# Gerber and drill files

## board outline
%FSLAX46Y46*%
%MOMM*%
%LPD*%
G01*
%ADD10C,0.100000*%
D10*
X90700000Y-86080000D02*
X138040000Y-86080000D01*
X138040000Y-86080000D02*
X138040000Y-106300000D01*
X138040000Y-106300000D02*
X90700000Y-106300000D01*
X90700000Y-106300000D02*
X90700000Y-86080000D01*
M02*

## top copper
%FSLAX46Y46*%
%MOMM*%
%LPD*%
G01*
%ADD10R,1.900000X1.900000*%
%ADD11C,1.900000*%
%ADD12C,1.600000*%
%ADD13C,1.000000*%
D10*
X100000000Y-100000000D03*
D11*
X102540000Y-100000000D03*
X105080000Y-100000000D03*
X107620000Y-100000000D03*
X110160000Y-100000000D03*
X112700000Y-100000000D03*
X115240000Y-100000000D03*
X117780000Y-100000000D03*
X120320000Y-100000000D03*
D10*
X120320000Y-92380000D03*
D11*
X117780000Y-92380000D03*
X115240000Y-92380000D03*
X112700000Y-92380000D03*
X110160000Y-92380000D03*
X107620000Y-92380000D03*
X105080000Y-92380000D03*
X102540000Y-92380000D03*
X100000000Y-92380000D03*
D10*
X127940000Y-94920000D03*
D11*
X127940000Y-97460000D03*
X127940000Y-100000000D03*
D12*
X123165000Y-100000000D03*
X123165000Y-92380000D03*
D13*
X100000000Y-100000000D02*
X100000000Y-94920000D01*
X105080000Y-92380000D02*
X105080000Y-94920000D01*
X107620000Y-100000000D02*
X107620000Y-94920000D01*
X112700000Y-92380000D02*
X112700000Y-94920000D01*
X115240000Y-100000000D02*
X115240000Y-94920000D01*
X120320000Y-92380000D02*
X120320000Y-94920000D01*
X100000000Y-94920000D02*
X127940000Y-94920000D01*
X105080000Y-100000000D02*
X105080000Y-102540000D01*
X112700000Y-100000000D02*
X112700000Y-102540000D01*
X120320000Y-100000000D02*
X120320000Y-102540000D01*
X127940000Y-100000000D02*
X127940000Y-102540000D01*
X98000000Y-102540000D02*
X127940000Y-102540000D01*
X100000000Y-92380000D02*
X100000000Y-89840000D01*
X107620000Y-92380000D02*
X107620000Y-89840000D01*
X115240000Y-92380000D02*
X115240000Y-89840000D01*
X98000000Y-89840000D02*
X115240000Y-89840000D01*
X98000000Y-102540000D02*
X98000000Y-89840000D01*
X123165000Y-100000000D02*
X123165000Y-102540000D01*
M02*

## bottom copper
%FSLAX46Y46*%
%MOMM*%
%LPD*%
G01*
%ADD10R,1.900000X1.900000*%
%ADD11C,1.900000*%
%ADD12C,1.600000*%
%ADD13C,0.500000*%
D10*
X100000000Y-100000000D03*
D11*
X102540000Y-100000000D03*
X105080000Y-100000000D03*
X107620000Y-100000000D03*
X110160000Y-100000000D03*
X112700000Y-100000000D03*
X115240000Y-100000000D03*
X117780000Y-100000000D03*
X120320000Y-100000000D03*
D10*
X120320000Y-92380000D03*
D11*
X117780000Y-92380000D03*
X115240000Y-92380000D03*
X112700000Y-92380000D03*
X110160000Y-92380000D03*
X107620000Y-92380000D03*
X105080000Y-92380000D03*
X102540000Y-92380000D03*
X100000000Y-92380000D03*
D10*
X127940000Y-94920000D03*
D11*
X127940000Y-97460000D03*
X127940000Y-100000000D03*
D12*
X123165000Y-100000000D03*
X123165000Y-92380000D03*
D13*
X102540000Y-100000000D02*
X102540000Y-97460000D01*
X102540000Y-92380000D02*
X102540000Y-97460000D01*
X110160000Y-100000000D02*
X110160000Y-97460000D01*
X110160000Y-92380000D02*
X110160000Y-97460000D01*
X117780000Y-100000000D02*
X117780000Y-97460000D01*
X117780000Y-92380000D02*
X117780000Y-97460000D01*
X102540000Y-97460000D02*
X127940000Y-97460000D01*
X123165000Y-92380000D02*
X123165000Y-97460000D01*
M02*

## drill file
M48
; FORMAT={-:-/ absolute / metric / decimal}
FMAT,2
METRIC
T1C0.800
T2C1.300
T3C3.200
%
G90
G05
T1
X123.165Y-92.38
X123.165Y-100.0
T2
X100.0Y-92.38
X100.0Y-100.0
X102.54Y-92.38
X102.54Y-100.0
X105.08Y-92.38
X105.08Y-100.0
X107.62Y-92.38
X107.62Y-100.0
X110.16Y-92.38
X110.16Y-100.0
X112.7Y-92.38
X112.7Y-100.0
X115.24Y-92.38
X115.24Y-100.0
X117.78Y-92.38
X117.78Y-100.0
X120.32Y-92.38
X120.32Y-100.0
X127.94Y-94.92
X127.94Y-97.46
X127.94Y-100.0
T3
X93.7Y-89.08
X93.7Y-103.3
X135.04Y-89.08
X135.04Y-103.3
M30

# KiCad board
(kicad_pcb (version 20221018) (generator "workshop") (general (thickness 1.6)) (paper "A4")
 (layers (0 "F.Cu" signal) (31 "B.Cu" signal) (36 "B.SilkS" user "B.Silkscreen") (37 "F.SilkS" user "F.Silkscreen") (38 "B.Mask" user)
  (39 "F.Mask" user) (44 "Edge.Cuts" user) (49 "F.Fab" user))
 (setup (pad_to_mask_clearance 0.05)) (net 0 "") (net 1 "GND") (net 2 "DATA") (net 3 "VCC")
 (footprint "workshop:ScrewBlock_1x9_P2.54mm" (layer "F.Cu") (at 100.000 100.000)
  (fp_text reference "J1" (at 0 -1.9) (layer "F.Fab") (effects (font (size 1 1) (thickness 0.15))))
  (pad "1" thru_hole rect (at 0.000 0) (size 1.9 1.9) (drill 1.3) (layers "*.Cu" "*.Mask") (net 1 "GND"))
  (pad "2" thru_hole circle (at 2.540 0) (size 1.9 1.9) (drill 1.3) (layers "*.Cu" "*.Mask") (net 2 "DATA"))
  (pad "3" thru_hole circle (at 5.080 0) (size 1.9 1.9) (drill 1.3) (layers "*.Cu" "*.Mask") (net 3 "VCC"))
  (pad "4" thru_hole circle (at 7.620 0) (size 1.9 1.9) (drill 1.3) (layers "*.Cu" "*.Mask") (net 1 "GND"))
  (pad "5" thru_hole circle (at 10.160 0) (size 1.9 1.9) (drill 1.3) (layers "*.Cu" "*.Mask") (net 2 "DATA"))
  (pad "6" thru_hole circle (at 12.700 0) (size 1.9 1.9) (drill 1.3) (layers "*.Cu" "*.Mask") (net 3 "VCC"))
  (pad "7" thru_hole circle (at 15.240 0) (size 1.9 1.9) (drill 1.3) (layers "*.Cu" "*.Mask") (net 1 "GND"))
  (pad "8" thru_hole circle (at 17.780 0) (size 1.9 1.9) (drill 1.3) (layers "*.Cu" "*.Mask") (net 2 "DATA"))
  (pad "9" thru_hole circle (at 20.320 0) (size 1.9 1.9) (drill 1.3) (layers "*.Cu" "*.Mask") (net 3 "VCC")))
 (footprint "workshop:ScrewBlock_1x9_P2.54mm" (layer "F.Cu") (at 120.320 92.380 180)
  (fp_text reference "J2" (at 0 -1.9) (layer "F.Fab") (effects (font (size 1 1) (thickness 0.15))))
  (pad "1" thru_hole rect (at 0.000 0) (size 1.9 1.9) (drill 1.3) (layers "*.Cu" "*.Mask") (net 1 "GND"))
  (pad "2" thru_hole circle (at 2.540 0) (size 1.9 1.9) (drill 1.3) (layers "*.Cu" "*.Mask") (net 2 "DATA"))
  (pad "3" thru_hole circle (at 5.080 0) (size 1.9 1.9) (drill 1.3) (layers "*.Cu" "*.Mask") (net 3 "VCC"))
  (pad "4" thru_hole circle (at 7.620 0) (size 1.9 1.9) (drill 1.3) (layers "*.Cu" "*.Mask") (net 1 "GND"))
  (pad "5" thru_hole circle (at 10.160 0) (size 1.9 1.9) (drill 1.3) (layers "*.Cu" "*.Mask") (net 2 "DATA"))
  (pad "6" thru_hole circle (at 12.700 0) (size 1.9 1.9) (drill 1.3) (layers "*.Cu" "*.Mask") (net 3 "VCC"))
  (pad "7" thru_hole circle (at 15.240 0) (size 1.9 1.9) (drill 1.3) (layers "*.Cu" "*.Mask") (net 1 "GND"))
  (pad "8" thru_hole circle (at 17.780 0) (size 1.9 1.9) (drill 1.3) (layers "*.Cu" "*.Mask") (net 2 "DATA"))
  (pad "9" thru_hole circle (at 20.320 0) (size 1.9 1.9) (drill 1.3) (layers "*.Cu" "*.Mask") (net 3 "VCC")))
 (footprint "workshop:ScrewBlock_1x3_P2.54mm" (layer "F.Cu") (at 127.940 94.920 270)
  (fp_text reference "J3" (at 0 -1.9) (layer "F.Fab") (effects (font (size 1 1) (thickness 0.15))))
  (pad "1" thru_hole rect (at 0.000 0) (size 1.9 1.9) (drill 1.3) (layers "*.Cu" "*.Mask") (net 1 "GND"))
  (pad "2" thru_hole circle (at 2.540 0) (size 1.9 1.9) (drill 1.3) (layers "*.Cu" "*.Mask") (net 2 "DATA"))
  (pad "3" thru_hole circle (at 5.080 0) (size 1.9 1.9) (drill 1.3) (layers "*.Cu" "*.Mask") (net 3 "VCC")))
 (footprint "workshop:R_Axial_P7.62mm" (layer "F.Cu") (at 123.165 100.000)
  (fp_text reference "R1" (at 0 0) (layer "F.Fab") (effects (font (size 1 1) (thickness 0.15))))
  (pad "1" thru_hole circle (at 0 0.000) (size 1.6 1.6) (drill 0.8) (layers "*.Cu" "*.Mask") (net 3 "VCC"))
  (pad "2" thru_hole circle (at 0 -7.620) (size 1.6 1.6) (drill 0.8) (layers "*.Cu" "*.Mask") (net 2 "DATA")))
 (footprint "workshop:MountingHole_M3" (layer "F.Cu") (at 93.700 89.080)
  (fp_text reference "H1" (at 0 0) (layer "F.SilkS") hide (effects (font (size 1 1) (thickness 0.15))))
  (pad "" np_thru_hole circle (at 0 0) (size 3.2 3.2) (drill 3.2) (layers "*.Cu" "*.Mask")))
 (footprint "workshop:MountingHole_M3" (layer "F.Cu") (at 93.700 103.300)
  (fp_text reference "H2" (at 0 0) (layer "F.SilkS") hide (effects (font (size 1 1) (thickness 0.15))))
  (pad "" np_thru_hole circle (at 0 0) (size 3.2 3.2) (drill 3.2) (layers "*.Cu" "*.Mask")))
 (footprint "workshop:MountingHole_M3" (layer "F.Cu") (at 135.040 89.080)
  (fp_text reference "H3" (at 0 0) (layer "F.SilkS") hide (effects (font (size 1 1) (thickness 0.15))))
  (pad "" np_thru_hole circle (at 0 0) (size 3.2 3.2) (drill 3.2) (layers "*.Cu" "*.Mask")))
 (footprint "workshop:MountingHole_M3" (layer "F.Cu") (at 135.040 103.300)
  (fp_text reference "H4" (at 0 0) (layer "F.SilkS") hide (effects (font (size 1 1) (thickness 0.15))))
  (pad "" np_thru_hole circle (at 0 0) (size 3.2 3.2) (drill 3.2) (layers "*.Cu" "*.Mask")))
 (segment (start 100.000 100.000) (end 100.000 94.920) (width 1.0) (layer "F.Cu") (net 1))
 (segment (start 105.080 92.380) (end 105.080 94.920) (width 1.0) (layer "F.Cu") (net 1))
 (segment (start 107.620 100.000) (end 107.620 94.920) (width 1.0) (layer "F.Cu") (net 1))
 (segment (start 112.700 92.380) (end 112.700 94.920) (width 1.0) (layer "F.Cu") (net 1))
 (segment (start 115.240 100.000) (end 115.240 94.920) (width 1.0) (layer "F.Cu") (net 1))
 (segment (start 120.320 92.380) (end 120.320 94.920) (width 1.0) (layer "F.Cu") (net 1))
 (segment (start 100.000 94.920) (end 127.940 94.920) (width 1.0) (layer "F.Cu") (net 1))
 (segment (start 102.540 100.000) (end 102.540 97.460) (width 0.5) (layer "B.Cu") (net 2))
 (segment (start 102.540 92.380) (end 102.540 97.460) (width 0.5) (layer "B.Cu") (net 2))
 (segment (start 110.160 100.000) (end 110.160 97.460) (width 0.5) (layer "B.Cu") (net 2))
 (segment (start 110.160 92.380) (end 110.160 97.460) (width 0.5) (layer "B.Cu") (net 2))
 (segment (start 117.780 100.000) (end 117.780 97.460) (width 0.5) (layer "B.Cu") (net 2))
 (segment (start 117.780 92.380) (end 117.780 97.460) (width 0.5) (layer "B.Cu") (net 2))
 (segment (start 102.540 97.460) (end 127.940 97.460) (width 0.5) (layer "B.Cu") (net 2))
 (segment (start 105.080 100.000) (end 105.080 102.540) (width 1.0) (layer "F.Cu") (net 3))
 (segment (start 112.700 100.000) (end 112.700 102.540) (width 1.0) (layer "F.Cu") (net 3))
 (segment (start 120.320 100.000) (end 120.320 102.540) (width 1.0) (layer "F.Cu") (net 3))
 (segment (start 127.940 100.000) (end 127.940 102.540) (width 1.0) (layer "F.Cu") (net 3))
 (segment (start 98.000 102.540) (end 127.940 102.540) (width 1.0) (layer "F.Cu") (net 3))
 (segment (start 100.000 92.380) (end 100.000 89.840) (width 1.0) (layer "F.Cu") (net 3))
 (segment (start 107.620 92.380) (end 107.620 89.840) (width 1.0) (layer "F.Cu") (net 3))
 (segment (start 115.240 92.380) (end 115.240 89.840) (width 1.0) (layer "F.Cu") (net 3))
 (segment (start 98.000 89.840) (end 115.240 89.840) (width 1.0) (layer "F.Cu") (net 3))
 (segment (start 98.000 102.540) (end 98.000 89.840) (width 1.0) (layer "F.Cu") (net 3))
 (segment (start 123.165 100.000) (end 123.165 102.540) (width 1.0) (layer "F.Cu") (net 3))
 (segment (start 123.165 92.380) (end 123.165 97.460) (width 0.5) (layer "B.Cu") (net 2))
 (gr_line (start 90.700 86.080) (end 138.040 86.080) (layer "Edge.Cuts") (width 0.1))
 (gr_line (start 138.040 86.080) (end 138.040 106.300) (layer "Edge.Cuts") (width 0.1))
 (gr_line (start 138.040 106.300) (end 90.700 106.300) (layer "Edge.Cuts") (width 0.1))
 (gr_line (start 90.700 106.300) (end 90.700 86.080) (layer "Edge.Cuts") (width 0.1)))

